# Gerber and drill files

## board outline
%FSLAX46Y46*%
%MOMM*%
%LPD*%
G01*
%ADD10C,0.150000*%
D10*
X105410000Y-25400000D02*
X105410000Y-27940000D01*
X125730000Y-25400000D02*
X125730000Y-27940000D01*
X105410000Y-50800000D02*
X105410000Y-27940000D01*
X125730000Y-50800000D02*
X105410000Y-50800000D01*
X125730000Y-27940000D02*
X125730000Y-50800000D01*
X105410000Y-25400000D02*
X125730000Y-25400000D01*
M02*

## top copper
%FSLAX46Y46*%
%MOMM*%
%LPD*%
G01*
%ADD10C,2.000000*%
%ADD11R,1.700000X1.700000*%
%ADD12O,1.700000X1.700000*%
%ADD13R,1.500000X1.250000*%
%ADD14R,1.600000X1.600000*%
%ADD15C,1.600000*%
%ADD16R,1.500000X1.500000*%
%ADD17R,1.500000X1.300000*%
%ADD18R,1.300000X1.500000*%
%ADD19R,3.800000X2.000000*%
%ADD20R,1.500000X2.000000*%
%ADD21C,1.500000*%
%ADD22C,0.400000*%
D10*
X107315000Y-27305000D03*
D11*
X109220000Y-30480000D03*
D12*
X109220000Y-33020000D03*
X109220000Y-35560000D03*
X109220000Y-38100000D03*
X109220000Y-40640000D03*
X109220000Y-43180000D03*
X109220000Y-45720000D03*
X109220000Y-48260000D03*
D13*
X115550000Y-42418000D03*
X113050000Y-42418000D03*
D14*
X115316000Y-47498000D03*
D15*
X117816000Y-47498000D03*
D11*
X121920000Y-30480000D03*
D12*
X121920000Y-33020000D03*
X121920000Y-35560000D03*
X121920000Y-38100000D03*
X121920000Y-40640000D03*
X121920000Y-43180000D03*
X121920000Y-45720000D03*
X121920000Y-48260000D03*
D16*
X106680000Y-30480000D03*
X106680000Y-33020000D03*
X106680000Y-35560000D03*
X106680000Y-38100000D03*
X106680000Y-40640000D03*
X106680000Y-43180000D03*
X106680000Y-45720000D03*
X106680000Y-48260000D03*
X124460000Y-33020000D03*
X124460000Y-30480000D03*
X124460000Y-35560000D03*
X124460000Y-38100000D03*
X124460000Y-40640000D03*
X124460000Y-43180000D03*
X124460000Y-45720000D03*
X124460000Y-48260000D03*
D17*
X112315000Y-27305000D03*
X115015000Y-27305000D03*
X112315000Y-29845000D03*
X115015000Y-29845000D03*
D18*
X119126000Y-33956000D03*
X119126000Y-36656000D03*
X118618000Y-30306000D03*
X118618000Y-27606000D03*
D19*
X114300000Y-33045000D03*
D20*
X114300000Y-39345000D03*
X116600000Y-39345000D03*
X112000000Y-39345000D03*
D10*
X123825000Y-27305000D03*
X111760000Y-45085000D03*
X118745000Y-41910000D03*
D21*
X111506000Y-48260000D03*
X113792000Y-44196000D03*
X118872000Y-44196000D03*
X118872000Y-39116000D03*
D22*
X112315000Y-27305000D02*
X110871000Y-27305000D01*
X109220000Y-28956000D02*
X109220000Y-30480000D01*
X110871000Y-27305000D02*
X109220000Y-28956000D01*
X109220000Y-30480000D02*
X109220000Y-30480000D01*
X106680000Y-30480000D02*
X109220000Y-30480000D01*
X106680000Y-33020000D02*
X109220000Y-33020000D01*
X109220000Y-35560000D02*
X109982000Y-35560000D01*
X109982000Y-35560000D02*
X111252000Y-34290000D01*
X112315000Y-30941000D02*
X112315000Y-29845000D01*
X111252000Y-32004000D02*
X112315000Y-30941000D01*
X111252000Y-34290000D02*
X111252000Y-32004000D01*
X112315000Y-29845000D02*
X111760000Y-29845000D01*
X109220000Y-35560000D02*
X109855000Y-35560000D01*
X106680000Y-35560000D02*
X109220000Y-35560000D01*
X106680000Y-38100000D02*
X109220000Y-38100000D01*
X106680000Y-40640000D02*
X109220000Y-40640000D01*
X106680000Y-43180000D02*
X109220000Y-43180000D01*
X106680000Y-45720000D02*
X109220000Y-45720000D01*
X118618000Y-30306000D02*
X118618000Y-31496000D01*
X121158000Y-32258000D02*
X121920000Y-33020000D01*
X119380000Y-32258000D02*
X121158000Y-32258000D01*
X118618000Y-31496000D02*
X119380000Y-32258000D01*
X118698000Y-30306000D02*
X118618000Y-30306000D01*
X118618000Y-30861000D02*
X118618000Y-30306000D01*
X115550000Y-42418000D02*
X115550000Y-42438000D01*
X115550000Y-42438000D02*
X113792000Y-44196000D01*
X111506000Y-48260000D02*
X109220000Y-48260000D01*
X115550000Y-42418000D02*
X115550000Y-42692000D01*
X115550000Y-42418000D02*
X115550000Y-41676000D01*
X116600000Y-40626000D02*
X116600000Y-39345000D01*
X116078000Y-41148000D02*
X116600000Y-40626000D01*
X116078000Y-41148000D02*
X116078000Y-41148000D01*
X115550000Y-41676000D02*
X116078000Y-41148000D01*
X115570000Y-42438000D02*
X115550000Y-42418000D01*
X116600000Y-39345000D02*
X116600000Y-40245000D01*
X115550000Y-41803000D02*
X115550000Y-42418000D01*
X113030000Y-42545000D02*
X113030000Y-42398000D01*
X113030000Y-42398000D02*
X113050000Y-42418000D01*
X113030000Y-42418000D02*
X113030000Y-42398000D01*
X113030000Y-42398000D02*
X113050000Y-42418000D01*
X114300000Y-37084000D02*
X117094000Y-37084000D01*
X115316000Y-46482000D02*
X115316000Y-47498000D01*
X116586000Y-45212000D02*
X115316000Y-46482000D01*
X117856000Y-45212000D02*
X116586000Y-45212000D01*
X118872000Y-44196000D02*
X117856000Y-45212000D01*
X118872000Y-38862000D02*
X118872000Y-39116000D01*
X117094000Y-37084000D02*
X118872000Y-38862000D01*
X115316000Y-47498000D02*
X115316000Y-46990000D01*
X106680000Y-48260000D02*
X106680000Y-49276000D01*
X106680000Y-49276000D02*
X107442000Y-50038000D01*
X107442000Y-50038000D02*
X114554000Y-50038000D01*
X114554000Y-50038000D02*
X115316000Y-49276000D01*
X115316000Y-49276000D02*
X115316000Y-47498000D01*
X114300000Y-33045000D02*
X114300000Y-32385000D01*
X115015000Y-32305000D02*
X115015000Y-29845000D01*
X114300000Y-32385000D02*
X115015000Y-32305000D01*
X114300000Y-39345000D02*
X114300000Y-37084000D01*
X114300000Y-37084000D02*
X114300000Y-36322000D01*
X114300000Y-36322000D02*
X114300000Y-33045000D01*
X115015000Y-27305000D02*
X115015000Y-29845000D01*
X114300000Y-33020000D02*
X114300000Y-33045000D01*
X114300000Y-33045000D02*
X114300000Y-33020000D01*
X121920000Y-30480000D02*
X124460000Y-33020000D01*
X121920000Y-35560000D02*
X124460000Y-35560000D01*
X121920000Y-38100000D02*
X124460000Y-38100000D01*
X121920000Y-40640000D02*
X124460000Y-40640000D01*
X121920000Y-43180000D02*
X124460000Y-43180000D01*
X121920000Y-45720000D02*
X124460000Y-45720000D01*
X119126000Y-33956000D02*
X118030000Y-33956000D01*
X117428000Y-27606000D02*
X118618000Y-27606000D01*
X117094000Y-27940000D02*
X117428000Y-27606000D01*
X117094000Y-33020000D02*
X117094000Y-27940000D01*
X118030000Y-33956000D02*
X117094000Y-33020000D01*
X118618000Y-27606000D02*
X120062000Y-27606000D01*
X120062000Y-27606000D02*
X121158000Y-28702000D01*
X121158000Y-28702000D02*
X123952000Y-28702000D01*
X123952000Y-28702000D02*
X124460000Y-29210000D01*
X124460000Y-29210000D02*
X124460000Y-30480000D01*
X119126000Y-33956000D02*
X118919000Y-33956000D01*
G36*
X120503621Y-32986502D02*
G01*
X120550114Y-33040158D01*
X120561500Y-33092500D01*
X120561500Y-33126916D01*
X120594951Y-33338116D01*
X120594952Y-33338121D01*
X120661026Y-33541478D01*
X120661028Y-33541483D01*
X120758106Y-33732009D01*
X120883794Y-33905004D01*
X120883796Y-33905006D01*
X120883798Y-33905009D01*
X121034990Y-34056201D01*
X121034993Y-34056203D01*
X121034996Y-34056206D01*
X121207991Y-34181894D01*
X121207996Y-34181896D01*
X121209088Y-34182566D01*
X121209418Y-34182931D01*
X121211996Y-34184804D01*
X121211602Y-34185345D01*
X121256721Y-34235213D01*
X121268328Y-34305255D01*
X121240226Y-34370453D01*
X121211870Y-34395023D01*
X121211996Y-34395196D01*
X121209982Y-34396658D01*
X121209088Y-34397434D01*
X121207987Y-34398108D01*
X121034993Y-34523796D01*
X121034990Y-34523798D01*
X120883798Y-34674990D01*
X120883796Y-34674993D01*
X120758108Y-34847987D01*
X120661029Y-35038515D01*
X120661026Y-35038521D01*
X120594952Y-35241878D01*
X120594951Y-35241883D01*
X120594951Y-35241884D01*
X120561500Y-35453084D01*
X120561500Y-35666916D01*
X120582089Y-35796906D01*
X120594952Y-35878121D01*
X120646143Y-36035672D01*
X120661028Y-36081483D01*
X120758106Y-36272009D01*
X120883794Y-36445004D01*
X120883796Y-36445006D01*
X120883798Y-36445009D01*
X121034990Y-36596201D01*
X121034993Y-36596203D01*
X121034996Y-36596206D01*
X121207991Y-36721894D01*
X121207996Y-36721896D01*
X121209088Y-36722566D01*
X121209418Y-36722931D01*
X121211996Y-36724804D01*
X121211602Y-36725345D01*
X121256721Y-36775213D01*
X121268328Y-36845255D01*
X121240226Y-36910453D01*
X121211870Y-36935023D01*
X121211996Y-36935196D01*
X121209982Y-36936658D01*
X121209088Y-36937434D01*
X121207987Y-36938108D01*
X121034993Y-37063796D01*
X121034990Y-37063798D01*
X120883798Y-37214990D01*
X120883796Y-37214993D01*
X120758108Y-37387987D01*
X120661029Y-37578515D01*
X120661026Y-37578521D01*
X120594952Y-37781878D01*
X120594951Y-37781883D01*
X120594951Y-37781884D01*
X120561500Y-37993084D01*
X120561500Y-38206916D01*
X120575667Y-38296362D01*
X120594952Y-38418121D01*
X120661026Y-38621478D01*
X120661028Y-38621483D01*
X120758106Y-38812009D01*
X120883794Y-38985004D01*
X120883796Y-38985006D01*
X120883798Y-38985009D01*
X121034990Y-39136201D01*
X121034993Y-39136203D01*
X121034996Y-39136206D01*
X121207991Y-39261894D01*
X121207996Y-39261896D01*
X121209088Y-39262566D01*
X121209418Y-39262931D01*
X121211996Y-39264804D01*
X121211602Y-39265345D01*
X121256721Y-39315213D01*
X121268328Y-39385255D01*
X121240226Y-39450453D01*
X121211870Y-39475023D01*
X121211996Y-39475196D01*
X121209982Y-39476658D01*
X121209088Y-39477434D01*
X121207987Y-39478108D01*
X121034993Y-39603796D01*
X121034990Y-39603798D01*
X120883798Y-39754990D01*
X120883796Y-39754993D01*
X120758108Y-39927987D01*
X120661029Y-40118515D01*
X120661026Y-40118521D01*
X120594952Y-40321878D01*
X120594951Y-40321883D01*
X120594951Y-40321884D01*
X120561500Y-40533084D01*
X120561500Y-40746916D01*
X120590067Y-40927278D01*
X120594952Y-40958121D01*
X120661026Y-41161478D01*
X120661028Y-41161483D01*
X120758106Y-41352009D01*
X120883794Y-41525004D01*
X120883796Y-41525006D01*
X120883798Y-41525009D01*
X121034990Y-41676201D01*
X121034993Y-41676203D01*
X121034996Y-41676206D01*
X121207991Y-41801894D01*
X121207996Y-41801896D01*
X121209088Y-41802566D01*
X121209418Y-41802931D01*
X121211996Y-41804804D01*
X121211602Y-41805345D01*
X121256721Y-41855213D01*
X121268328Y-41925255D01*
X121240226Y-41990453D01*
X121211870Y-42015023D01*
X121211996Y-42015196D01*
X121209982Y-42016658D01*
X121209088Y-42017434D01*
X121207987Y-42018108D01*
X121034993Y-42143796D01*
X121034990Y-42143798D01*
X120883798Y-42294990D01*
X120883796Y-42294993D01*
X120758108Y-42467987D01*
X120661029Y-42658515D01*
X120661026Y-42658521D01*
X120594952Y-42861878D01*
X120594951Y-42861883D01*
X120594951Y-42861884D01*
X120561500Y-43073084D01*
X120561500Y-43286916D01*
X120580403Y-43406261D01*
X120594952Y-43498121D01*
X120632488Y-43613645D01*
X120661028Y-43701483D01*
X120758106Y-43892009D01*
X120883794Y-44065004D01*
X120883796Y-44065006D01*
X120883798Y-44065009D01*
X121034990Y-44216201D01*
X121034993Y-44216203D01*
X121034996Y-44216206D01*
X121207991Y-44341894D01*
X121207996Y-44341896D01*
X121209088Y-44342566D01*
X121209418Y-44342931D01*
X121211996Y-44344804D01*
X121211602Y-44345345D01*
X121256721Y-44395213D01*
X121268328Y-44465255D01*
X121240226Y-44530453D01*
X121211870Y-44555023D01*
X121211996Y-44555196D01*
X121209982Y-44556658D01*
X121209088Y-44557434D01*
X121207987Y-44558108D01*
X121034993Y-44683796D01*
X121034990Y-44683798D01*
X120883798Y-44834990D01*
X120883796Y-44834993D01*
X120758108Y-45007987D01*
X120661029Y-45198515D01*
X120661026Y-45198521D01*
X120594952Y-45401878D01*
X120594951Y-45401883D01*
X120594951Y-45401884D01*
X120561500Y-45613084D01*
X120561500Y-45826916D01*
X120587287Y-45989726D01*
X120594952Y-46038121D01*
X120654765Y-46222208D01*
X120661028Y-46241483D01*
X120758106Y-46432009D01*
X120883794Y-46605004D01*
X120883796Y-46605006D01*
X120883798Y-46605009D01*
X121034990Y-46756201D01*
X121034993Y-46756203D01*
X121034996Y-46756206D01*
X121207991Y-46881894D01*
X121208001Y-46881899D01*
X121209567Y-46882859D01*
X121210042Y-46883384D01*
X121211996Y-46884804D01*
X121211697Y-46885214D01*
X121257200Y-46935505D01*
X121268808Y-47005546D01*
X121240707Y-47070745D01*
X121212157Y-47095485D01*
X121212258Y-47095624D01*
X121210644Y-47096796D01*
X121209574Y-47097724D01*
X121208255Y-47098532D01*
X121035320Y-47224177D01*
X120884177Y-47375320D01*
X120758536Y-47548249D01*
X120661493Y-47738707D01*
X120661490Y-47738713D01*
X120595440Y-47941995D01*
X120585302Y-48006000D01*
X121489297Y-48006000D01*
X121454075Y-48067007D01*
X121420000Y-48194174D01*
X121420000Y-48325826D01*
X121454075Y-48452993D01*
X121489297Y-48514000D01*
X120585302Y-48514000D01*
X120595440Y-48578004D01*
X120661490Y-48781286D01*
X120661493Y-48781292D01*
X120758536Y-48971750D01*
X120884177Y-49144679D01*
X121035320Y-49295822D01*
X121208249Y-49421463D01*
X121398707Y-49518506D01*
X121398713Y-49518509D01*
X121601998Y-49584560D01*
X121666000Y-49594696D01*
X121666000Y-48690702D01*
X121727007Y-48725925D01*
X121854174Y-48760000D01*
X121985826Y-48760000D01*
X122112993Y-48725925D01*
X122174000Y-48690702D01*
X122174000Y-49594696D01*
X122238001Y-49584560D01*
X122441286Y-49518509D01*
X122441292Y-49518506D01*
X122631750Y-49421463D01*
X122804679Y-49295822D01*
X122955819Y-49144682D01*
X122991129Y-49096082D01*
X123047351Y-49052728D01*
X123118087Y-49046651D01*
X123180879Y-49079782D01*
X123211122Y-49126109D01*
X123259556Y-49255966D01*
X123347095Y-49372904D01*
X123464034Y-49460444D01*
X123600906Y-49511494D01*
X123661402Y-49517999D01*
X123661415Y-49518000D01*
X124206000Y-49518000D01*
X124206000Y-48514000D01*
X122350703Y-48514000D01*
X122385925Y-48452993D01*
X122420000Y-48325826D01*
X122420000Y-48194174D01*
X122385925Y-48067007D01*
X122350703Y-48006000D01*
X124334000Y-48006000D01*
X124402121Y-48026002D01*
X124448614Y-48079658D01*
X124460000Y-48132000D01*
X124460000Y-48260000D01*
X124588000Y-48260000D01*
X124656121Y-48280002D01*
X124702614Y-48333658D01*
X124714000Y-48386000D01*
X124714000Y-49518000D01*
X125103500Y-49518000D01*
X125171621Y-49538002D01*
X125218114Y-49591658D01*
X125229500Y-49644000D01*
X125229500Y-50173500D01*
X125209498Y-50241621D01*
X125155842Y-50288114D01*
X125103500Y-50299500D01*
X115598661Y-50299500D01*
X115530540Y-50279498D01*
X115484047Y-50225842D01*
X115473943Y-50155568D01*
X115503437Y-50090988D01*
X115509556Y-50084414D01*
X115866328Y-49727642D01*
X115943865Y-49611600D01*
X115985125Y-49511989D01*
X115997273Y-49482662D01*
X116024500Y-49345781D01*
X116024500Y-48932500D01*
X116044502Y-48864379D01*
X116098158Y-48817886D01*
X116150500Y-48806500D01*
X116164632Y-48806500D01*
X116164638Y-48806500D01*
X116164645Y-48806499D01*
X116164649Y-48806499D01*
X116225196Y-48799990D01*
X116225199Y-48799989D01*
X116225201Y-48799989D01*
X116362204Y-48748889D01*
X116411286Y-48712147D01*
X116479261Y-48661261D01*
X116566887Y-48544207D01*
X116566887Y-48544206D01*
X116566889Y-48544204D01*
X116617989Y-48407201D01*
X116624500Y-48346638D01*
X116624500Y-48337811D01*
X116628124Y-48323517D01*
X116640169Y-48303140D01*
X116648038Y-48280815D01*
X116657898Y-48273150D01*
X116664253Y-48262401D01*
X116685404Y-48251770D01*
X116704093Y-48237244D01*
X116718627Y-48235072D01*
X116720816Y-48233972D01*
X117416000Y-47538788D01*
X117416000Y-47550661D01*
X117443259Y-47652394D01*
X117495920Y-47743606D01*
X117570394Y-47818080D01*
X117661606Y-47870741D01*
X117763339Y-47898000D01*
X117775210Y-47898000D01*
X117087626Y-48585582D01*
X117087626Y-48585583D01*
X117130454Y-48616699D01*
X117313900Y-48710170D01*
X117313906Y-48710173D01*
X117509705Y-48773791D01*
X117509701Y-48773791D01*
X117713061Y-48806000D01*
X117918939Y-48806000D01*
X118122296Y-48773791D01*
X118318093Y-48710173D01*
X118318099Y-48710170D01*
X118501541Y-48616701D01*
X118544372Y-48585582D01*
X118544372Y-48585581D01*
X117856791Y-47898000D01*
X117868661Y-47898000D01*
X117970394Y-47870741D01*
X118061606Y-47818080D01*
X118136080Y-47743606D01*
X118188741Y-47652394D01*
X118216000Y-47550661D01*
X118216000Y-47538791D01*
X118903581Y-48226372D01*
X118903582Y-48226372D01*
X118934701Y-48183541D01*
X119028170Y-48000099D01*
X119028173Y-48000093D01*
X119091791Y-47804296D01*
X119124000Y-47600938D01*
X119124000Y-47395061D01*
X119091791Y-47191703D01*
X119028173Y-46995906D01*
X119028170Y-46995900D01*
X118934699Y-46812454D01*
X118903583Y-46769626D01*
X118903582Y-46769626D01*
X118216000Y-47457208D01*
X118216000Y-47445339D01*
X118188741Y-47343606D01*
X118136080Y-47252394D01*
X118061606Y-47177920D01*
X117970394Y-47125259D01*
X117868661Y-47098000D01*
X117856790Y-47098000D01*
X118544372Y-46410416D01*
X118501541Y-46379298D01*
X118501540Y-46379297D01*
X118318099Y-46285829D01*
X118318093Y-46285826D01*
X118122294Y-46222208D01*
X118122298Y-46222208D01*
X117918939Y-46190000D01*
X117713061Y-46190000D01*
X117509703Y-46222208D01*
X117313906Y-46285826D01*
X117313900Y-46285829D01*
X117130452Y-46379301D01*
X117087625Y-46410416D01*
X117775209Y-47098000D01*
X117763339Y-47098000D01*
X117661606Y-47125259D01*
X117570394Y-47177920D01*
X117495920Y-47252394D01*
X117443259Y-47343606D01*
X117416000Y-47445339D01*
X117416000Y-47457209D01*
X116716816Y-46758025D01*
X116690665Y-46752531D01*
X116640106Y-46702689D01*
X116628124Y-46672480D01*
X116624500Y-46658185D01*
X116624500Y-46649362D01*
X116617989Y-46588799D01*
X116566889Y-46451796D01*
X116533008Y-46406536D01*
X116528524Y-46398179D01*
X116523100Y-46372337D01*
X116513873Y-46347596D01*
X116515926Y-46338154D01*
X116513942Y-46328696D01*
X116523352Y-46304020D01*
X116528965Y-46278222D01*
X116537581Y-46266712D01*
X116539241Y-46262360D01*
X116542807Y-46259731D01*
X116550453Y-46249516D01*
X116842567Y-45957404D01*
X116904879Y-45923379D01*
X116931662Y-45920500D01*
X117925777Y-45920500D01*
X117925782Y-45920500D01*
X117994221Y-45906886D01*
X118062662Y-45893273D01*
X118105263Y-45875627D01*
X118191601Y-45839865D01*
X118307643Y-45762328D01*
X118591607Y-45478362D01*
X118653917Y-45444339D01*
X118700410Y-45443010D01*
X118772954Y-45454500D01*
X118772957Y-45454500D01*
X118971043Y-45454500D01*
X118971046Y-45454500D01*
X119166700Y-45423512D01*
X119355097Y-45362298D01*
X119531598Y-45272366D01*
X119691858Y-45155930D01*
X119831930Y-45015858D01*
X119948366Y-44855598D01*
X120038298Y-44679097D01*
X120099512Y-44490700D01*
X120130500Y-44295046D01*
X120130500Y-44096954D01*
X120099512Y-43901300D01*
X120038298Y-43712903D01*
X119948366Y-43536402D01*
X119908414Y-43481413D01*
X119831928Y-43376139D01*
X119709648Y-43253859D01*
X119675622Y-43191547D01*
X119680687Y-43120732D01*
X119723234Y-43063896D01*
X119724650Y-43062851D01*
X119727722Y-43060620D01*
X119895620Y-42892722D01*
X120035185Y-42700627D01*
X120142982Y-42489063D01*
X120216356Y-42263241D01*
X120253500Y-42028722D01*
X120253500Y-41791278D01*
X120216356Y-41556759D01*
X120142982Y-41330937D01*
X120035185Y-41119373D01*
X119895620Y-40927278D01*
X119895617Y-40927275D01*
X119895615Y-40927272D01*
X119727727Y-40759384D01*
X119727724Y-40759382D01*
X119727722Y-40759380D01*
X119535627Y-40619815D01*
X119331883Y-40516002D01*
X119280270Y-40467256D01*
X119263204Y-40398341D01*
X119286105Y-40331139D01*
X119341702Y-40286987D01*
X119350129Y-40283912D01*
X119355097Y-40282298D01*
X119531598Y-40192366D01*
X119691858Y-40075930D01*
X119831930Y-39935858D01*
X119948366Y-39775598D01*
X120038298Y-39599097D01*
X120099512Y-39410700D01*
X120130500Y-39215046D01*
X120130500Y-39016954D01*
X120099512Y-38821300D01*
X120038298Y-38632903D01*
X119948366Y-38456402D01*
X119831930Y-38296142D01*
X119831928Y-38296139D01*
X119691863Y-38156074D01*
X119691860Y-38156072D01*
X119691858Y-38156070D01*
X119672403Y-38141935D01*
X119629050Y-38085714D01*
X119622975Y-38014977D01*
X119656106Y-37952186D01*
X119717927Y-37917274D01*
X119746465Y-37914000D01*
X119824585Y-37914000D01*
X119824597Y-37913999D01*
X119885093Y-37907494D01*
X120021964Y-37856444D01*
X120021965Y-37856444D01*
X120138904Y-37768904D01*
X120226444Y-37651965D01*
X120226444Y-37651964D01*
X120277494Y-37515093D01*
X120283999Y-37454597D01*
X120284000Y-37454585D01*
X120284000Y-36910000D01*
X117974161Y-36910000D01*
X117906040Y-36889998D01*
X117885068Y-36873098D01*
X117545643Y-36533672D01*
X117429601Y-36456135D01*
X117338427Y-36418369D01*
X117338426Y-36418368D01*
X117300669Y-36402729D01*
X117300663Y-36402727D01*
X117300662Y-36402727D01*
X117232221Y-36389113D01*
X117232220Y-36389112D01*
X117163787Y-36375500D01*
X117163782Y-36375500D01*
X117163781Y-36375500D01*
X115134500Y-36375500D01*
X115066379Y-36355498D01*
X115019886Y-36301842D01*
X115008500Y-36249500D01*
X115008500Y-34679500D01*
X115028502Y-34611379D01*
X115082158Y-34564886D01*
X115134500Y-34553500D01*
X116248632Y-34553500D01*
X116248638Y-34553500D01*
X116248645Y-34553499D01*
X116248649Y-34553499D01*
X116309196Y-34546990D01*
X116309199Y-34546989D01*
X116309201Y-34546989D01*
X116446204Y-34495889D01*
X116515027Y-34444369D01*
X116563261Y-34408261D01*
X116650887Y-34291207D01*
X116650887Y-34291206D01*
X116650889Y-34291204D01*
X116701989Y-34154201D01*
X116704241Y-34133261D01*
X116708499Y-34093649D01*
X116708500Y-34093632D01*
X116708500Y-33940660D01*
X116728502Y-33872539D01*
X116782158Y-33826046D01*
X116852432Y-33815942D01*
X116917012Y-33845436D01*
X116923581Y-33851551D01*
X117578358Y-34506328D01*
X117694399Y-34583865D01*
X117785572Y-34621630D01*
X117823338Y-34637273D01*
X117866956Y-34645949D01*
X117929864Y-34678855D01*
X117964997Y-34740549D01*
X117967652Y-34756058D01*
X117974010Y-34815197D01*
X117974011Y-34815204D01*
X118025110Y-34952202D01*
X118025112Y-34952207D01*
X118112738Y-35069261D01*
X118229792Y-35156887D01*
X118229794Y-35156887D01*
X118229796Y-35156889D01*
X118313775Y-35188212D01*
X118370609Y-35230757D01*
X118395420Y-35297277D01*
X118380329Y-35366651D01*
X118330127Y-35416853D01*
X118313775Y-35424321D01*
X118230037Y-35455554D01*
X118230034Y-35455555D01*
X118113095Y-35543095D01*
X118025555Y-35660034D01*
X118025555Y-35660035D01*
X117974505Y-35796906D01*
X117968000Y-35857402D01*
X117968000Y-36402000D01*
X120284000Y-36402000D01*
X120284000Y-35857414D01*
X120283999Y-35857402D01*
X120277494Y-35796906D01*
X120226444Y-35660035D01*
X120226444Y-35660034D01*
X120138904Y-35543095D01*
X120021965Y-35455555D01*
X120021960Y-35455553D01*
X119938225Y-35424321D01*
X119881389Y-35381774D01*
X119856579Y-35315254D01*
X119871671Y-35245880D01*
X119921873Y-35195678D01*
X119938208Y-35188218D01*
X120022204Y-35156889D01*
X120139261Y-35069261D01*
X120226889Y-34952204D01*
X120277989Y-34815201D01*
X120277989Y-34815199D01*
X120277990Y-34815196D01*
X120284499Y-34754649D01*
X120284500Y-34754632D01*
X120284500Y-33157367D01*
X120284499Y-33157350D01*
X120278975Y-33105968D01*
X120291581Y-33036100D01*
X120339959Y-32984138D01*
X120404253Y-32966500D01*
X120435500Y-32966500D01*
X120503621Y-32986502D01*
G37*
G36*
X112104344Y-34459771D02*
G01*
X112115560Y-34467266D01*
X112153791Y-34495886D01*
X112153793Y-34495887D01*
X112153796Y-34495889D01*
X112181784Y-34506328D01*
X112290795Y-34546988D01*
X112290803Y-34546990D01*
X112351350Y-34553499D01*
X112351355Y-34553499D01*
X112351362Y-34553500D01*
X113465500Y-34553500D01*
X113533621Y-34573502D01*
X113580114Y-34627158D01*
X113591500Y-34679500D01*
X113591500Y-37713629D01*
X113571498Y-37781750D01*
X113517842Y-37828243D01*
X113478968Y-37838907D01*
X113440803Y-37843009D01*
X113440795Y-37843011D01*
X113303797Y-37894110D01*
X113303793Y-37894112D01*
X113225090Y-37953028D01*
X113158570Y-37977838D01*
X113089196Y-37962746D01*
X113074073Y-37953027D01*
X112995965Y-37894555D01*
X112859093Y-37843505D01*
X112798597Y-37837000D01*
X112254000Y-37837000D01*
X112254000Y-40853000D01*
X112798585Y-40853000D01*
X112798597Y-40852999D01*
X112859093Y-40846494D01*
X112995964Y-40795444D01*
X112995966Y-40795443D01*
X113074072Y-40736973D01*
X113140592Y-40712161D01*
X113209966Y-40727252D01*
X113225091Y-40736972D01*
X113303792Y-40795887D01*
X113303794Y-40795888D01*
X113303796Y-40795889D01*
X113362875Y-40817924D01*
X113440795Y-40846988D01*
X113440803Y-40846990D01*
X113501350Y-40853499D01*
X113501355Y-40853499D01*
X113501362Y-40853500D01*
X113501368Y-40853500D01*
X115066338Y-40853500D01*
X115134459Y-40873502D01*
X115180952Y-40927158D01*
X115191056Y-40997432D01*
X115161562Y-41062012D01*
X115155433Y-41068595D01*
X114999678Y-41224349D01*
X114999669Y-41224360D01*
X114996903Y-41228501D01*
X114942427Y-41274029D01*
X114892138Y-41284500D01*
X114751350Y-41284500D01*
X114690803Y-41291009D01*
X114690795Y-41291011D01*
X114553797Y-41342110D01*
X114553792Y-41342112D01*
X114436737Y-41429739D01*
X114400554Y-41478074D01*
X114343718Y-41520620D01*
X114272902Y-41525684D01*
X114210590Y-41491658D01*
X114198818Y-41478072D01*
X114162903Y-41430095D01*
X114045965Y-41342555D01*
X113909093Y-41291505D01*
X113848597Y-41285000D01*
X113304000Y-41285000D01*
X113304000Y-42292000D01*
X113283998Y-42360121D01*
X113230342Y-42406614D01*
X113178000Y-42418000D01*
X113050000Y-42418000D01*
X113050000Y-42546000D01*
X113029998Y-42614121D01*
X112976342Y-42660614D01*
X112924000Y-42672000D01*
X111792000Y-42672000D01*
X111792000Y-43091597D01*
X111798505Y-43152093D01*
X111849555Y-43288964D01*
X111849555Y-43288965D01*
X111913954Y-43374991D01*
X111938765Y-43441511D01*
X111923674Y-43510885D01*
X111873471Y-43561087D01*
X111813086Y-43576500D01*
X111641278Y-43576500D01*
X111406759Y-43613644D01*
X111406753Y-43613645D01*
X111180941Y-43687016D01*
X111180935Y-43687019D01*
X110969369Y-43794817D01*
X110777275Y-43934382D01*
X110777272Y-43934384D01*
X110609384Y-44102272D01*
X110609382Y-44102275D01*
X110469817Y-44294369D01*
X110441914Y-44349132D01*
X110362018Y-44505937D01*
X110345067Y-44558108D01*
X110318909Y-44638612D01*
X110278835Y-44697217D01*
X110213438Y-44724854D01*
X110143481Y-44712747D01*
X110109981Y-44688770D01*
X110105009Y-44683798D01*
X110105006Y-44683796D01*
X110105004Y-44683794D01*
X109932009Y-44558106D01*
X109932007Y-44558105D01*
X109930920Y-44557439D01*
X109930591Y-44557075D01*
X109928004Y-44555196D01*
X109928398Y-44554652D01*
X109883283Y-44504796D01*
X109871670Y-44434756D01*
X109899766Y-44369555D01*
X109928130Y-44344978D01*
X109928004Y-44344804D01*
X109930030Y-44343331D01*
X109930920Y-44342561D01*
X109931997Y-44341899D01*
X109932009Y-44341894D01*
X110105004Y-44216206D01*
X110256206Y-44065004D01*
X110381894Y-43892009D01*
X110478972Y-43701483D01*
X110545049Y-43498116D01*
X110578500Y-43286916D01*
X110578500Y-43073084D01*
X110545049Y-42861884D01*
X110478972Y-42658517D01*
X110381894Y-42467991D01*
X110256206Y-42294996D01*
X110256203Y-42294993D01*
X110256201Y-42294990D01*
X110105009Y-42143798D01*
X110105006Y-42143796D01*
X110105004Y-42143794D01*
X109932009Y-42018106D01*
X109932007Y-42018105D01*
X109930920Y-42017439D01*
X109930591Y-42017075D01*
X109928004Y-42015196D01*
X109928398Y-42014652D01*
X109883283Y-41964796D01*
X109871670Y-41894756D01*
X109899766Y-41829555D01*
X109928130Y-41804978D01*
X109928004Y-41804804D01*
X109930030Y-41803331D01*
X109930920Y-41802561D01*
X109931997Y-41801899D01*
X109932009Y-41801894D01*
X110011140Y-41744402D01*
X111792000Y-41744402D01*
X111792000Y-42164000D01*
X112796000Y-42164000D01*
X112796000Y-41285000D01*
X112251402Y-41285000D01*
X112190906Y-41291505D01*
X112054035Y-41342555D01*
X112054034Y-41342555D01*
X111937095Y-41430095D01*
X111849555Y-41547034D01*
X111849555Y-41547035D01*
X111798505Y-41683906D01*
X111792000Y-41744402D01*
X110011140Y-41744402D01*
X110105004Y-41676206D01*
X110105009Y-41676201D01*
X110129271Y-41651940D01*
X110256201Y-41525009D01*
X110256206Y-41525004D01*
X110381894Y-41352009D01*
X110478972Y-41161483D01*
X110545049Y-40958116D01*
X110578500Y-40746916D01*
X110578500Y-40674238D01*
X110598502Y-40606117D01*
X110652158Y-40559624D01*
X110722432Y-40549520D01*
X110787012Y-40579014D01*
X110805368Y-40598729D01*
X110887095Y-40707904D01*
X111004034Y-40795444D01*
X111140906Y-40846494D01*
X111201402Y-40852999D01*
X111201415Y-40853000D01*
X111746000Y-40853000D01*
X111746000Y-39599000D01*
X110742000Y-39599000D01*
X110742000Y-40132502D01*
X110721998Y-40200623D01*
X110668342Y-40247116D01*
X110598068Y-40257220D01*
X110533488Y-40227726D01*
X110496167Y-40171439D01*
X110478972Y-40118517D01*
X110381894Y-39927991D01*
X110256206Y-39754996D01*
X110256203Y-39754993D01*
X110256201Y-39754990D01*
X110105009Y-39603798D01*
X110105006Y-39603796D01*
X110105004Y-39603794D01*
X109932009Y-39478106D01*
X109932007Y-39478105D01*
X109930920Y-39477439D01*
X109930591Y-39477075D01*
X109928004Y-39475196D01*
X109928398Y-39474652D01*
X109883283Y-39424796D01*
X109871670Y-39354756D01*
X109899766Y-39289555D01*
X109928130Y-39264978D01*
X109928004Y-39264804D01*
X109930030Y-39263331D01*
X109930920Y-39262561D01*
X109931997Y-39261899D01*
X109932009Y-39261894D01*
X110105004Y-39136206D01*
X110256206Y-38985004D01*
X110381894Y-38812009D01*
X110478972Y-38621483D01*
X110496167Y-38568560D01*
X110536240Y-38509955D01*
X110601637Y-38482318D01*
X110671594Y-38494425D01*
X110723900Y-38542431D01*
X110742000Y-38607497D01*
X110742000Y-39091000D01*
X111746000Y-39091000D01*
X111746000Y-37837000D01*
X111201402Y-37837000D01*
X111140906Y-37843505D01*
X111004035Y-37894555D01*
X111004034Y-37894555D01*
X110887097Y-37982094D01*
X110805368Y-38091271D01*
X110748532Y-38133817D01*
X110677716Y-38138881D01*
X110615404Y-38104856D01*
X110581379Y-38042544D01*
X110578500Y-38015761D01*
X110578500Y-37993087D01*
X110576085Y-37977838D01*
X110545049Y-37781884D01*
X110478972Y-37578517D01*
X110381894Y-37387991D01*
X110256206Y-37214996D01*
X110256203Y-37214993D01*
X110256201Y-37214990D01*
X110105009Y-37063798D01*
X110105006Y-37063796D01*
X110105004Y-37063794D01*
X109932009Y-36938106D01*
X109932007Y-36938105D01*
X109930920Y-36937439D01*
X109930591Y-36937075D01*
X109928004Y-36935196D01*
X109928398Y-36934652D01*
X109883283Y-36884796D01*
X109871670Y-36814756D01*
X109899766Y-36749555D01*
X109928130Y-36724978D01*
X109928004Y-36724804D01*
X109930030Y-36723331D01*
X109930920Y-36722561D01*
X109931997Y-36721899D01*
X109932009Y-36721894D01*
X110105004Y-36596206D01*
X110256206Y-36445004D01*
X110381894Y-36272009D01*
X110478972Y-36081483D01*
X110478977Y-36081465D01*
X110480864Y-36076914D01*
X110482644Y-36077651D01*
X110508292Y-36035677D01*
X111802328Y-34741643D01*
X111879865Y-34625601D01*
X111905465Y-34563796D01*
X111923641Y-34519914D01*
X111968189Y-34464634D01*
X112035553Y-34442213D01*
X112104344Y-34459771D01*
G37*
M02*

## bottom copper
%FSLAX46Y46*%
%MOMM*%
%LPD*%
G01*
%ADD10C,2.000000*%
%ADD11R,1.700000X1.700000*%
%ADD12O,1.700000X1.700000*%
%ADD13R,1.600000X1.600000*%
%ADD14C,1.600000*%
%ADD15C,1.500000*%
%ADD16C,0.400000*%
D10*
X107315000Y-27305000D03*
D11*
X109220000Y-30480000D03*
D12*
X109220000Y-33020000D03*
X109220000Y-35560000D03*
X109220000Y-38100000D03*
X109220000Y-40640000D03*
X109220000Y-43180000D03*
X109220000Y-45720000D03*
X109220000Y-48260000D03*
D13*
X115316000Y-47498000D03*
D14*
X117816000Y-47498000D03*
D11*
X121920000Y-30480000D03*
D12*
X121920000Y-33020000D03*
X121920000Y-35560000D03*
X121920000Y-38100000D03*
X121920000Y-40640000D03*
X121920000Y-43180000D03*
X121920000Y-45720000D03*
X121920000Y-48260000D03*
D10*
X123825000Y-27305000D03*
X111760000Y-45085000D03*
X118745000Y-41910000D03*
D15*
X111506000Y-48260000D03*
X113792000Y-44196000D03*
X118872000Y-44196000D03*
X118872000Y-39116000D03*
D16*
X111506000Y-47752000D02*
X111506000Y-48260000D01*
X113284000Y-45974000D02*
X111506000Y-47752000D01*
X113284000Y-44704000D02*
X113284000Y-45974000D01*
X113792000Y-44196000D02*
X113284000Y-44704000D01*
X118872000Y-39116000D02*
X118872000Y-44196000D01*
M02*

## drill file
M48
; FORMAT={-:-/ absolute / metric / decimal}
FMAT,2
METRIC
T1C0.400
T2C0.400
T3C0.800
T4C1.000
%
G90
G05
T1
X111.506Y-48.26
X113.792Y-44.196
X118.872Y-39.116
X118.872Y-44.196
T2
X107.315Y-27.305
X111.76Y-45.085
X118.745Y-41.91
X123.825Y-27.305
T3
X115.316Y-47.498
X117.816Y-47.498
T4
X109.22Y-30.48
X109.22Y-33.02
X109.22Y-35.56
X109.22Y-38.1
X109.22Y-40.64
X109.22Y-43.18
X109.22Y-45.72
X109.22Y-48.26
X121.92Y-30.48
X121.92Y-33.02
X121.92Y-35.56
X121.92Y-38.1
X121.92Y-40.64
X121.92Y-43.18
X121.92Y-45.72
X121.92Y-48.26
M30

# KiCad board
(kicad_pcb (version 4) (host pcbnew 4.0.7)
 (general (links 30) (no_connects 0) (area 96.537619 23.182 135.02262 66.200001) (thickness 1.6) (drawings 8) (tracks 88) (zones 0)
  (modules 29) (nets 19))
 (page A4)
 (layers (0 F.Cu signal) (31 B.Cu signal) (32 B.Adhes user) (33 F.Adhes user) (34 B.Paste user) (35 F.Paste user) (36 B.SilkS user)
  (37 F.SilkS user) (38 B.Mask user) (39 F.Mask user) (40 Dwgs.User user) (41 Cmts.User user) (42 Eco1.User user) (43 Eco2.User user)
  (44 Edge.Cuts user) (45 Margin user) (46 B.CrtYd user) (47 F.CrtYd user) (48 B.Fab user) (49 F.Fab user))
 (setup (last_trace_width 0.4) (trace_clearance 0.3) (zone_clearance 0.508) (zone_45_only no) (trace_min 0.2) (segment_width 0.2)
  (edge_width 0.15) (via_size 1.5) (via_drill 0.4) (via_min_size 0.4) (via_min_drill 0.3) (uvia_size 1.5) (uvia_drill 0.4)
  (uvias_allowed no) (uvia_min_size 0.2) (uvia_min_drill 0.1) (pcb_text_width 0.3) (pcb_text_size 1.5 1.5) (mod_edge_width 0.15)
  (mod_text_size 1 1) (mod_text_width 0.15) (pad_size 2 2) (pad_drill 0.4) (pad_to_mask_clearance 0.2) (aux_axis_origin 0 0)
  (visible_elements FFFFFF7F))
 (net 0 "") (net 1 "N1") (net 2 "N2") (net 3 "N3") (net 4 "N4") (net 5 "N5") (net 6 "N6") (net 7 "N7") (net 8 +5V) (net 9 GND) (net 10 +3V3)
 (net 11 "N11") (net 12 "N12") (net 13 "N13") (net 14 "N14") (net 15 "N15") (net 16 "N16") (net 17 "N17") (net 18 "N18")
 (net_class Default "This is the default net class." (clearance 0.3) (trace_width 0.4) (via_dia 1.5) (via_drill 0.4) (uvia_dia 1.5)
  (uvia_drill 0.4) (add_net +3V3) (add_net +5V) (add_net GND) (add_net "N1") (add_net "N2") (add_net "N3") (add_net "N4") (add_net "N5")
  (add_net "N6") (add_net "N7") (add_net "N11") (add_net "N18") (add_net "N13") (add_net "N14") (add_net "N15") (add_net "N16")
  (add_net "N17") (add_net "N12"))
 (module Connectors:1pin (layer F.Cu) (at 107.315 27.305)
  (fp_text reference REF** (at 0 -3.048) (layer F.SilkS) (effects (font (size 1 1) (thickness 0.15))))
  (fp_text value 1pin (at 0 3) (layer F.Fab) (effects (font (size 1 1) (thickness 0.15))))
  (pad 1 thru_hole circle (at 0 0) (size 2 2) (drill 0.4) (layers *.Cu *.Mask)))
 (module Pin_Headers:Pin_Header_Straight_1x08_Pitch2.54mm (layer F.Cu) (at 109.22 30.48)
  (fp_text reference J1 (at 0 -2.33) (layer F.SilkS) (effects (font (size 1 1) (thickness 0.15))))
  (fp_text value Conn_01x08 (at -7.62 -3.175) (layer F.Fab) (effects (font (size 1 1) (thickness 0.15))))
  (pad 1 thru_hole rect (at 0 0) (size 1.7 1.7) (drill 1) (layers *.Cu *.Mask) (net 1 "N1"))
  (pad 2 thru_hole oval (at 0 2.54) (size 1.7 1.7) (drill 1) (layers *.Cu *.Mask) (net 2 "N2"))
  (pad 3 thru_hole oval (at 0 5.08) (size 1.7 1.7) (drill 1) (layers *.Cu *.Mask) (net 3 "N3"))
  (pad 4 thru_hole oval (at 0 7.62) (size 1.7 1.7) (drill 1) (layers *.Cu *.Mask) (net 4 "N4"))
  (pad 5 thru_hole oval (at 0 10.16) (size 1.7 1.7) (drill 1) (layers *.Cu *.Mask) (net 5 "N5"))
  (pad 6 thru_hole oval (at 0 12.7) (size 1.7 1.7) (drill 1) (layers *.Cu *.Mask) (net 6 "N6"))
  (pad 7 thru_hole oval (at 0 15.24) (size 1.7 1.7) (drill 1) (layers *.Cu *.Mask) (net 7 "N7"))
  (pad 8 thru_hole oval (at 0 17.78) (size 1.7 1.7) (drill 1) (layers *.Cu *.Mask) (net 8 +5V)))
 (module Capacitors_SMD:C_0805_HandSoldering (layer F.Cu) (at 114.3 42.418 180)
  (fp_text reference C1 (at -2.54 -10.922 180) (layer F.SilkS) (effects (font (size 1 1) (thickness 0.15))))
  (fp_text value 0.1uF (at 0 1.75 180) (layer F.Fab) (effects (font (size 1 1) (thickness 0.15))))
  (pad 1 smd rect (at -1.25 0 180) (size 1.5 1.25) (layers F.Cu F.Paste F.Mask) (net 8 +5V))
  (pad 2 smd rect (at 1.25 0 180) (size 1.5 1.25) (layers F.Cu F.Paste F.Mask) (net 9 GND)))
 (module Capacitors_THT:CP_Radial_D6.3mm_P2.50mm (layer F.Cu) (at 115.316 47.498)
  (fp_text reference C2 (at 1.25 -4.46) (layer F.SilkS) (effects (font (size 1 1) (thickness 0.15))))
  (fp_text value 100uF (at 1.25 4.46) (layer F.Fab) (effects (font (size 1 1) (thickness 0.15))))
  (pad 1 thru_hole rect (at 0 0) (size 1.6 1.6) (drill 0.8) (layers *.Cu *.Mask) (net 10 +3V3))
  (pad 2 thru_hole circle (at 2.5 0) (size 1.6 1.6) (drill 0.8) (layers *.Cu *.Mask) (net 9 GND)))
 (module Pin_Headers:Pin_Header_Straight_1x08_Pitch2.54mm (layer F.Cu) (at 121.92 30.48)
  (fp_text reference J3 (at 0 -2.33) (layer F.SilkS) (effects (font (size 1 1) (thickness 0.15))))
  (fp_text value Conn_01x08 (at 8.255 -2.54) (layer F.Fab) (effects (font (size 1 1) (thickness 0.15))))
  (pad 1 thru_hole rect (at 0 0) (size 1.7 1.7) (drill 1) (layers *.Cu *.Mask) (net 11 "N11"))
  (pad 2 thru_hole oval (at 0 2.54) (size 1.7 1.7) (drill 1) (layers *.Cu *.Mask) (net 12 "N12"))
  (pad 3 thru_hole oval (at 0 5.08) (size 1.7 1.7) (drill 1) (layers *.Cu *.Mask) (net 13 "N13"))
  (pad 4 thru_hole oval (at 0 7.62) (size 1.7 1.7) (drill 1) (layers *.Cu *.Mask) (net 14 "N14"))
  (pad 5 thru_hole oval (at 0 10.16) (size 1.7 1.7) (drill 1) (layers *.Cu *.Mask) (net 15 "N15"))
  (pad 6 thru_hole oval (at 0 12.7) (size 1.7 1.7) (drill 1) (layers *.Cu *.Mask) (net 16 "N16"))
  (pad 7 thru_hole oval (at 0 15.24) (size 1.7 1.7) (drill 1) (layers *.Cu *.Mask) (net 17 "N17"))
  (pad 8 thru_hole oval (at 0 17.78) (size 1.7 1.7) (drill 1) (layers *.Cu *.Mask) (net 9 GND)))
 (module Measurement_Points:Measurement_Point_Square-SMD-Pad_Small (layer F.Cu) (at 106.68 30.48)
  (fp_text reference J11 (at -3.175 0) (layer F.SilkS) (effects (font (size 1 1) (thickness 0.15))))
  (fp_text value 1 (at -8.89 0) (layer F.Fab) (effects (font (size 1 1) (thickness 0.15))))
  (pad 1 smd rect (at 0 0) (size 1.5 1.5) (layers F.Cu F.Mask) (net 1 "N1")))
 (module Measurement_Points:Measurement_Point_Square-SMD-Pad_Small (layer F.Cu) (at 106.68 33.02)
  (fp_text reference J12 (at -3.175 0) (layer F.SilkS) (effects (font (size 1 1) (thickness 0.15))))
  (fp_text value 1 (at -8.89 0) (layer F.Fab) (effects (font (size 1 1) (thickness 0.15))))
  (pad 1 smd rect (at 0 0) (size 1.5 1.5) (layers F.Cu F.Mask) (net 2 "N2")))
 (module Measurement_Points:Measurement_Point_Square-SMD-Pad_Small (layer F.Cu) (at 106.68 35.56)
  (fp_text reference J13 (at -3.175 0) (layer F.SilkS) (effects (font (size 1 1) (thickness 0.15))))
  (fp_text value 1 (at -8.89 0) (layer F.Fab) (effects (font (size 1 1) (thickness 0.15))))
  (pad 1 smd rect (at 0 0) (size 1.5 1.5) (layers F.Cu F.Mask) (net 3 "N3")))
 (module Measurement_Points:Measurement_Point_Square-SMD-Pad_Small (layer F.Cu) (at 106.68 38.1)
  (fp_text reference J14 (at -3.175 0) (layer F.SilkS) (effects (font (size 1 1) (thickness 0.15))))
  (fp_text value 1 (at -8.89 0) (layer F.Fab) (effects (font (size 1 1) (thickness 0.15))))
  (pad 1 smd rect (at 0 0) (size 1.5 1.5) (layers F.Cu F.Mask) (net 4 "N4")))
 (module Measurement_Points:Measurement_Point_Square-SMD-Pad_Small (layer F.Cu) (at 106.68 40.64)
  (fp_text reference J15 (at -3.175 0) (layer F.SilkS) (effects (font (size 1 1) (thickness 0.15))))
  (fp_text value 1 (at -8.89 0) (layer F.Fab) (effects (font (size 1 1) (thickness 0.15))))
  (pad 1 smd rect (at 0 0) (size 1.5 1.5) (layers F.Cu F.Mask) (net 5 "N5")))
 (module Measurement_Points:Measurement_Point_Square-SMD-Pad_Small (layer F.Cu) (at 106.68 43.18)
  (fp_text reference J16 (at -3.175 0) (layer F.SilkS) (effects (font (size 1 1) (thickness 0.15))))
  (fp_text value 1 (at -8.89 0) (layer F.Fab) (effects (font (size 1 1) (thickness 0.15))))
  (pad 1 smd rect (at 0 0) (size 1.5 1.5) (layers F.Cu F.Mask) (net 6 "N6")))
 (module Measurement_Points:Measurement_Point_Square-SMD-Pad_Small (layer F.Cu) (at 106.68 45.72)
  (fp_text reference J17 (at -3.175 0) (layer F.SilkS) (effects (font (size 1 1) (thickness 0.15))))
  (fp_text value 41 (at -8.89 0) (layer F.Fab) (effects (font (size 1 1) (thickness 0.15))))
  (pad 1 smd rect (at 0 0) (size 1.5 1.5) (layers F.Cu F.Mask) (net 7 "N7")))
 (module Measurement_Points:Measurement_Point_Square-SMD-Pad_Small (layer F.Cu) (at 106.68 48.26)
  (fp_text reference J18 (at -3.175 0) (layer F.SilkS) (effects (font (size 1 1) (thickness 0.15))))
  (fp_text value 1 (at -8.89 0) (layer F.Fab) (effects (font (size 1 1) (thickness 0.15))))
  (pad 1 smd rect (at 0 0) (size 1.5 1.5) (layers F.Cu F.Mask) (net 10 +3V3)))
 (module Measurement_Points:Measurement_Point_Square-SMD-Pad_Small (layer F.Cu) (at 124.46 33.02)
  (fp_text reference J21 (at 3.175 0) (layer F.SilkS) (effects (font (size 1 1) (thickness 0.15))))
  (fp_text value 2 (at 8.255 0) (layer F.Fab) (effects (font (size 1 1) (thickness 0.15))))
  (pad 1 smd rect (at 0 0) (size 1.5 1.5) (layers F.Cu F.Mask) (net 11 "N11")))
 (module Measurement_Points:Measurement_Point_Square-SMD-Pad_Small (layer F.Cu) (at 124.46 30.48)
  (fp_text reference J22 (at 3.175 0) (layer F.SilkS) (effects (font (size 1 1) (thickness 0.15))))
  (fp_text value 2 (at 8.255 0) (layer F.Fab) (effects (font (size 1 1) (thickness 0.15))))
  (pad 1 smd rect (at 0 0) (size 1.5 1.5) (layers F.Cu F.Mask) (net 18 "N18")))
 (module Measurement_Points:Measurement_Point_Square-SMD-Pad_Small (layer F.Cu) (at 124.46 35.56)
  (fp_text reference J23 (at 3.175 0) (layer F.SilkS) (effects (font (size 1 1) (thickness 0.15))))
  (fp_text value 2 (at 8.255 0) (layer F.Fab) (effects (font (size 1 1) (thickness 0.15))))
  (pad 1 smd rect (at 0 0) (size 1.5 1.5) (layers F.Cu F.Mask) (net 13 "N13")))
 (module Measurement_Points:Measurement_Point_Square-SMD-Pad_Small (layer F.Cu) (at 124.46 38.1)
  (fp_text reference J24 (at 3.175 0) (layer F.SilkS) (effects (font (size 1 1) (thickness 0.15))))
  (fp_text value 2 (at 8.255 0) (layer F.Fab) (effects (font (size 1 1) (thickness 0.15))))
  (pad 1 smd rect (at 0 0) (size 1.5 1.5) (layers F.Cu F.Mask) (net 14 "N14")))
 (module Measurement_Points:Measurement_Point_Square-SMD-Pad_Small (layer F.Cu) (at 124.46 40.64)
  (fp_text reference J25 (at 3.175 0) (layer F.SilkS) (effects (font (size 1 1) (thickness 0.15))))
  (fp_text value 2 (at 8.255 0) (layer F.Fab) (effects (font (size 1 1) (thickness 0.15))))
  (pad 1 smd rect (at 0 0) (size 1.5 1.5) (layers F.Cu F.Mask) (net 15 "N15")))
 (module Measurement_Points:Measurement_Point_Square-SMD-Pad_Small (layer F.Cu) (at 124.46 43.18)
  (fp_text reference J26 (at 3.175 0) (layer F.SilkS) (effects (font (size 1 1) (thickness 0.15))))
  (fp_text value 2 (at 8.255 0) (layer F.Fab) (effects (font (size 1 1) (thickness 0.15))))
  (pad 1 smd rect (at 0 0) (size 1.5 1.5) (layers F.Cu F.Mask) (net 16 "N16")))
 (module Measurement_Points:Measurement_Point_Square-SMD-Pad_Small (layer F.Cu) (at 124.46 45.72)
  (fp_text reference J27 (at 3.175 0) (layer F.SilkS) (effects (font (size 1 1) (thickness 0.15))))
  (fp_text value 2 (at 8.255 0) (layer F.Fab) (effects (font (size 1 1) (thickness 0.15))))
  (pad 1 smd rect (at 0 0) (size 1.5 1.5) (layers F.Cu F.Mask) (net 17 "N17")))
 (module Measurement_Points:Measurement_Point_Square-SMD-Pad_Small (layer F.Cu) (at 124.46 48.26)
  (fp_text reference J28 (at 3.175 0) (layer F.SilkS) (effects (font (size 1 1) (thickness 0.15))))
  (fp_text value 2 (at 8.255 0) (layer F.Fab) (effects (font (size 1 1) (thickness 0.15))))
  (pad 1 smd rect (at 0 0) (size 1.5 1.5) (layers F.Cu F.Mask) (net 9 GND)))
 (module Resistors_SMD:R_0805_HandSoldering (layer F.Cu) (at 113.665 27.305)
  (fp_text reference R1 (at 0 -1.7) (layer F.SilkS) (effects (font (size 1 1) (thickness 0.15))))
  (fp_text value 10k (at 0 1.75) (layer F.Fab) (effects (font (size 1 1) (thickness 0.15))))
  (pad 1 smd rect (at -1.35 0) (size 1.5 1.3) (layers F.Cu F.Paste F.Mask) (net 1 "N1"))
  (pad 2 smd rect (at 1.35 0) (size 1.5 1.3) (layers F.Cu F.Paste F.Mask) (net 10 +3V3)))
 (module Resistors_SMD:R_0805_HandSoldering (layer F.Cu) (at 113.665 29.845)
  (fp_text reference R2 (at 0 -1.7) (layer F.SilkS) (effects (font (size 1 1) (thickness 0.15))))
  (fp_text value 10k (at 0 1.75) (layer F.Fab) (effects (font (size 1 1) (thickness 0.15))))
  (pad 1 smd rect (at -1.35 0) (size 1.5 1.3) (layers F.Cu F.Paste F.Mask) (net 3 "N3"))
  (pad 2 smd rect (at 1.35 0) (size 1.5 1.3) (layers F.Cu F.Paste F.Mask) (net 10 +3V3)))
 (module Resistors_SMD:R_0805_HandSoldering (layer F.Cu) (at 119.126 35.306 270)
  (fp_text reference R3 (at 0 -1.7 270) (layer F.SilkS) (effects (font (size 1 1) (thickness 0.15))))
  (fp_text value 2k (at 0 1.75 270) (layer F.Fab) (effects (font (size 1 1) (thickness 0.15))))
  (pad 1 smd rect (at -1.35 0 270) (size 1.5 1.3) (layers F.Cu F.Paste F.Mask) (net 18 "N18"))
  (pad 2 smd rect (at 1.35 0 270) (size 1.5 1.3) (layers F.Cu F.Paste F.Mask) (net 9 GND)))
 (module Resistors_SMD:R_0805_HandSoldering (layer F.Cu) (at 118.618 28.956 90)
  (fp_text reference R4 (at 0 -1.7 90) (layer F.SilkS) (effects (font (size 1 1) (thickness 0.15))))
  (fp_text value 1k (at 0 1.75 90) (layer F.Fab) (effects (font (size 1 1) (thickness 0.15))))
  (pad 1 smd rect (at -1.35 0 90) (size 1.5 1.3) (layers F.Cu F.Paste F.Mask) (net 12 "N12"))
  (pad 2 smd rect (at 1.35 0 90) (size 1.5 1.3) (layers F.Cu F.Paste F.Mask) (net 18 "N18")))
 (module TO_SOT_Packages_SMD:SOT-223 (layer F.Cu) (at 114.3 36.195 90)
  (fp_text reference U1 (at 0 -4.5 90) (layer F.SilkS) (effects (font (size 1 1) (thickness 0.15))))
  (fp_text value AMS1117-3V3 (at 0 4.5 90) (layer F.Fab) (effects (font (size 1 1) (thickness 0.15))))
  (pad 4 smd rect (at 3.15 0 90) (size 2 3.8) (layers F.Cu F.Paste F.Mask) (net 10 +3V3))
  (pad 2 smd rect (at -3.15 0 90) (size 2 1.5) (layers F.Cu F.Paste F.Mask) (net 10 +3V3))
  (pad 3 smd rect (at -3.15 2.3 90) (size 2 1.5) (layers F.Cu F.Paste F.Mask) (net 8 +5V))
  (pad 1 smd rect (at -3.15 -2.3 90) (size 2 1.5) (layers F.Cu F.Paste F.Mask) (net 9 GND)))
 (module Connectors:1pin (layer F.Cu) (at 123.825 27.305)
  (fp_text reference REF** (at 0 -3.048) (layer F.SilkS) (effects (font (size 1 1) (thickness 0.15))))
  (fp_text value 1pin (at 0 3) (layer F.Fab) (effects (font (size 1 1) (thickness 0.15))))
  (pad 1 thru_hole circle (at 0 0) (size 2 2) (drill 0.4) (layers *.Cu *.Mask)))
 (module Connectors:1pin (layer F.Cu) (at 111.76 45.085)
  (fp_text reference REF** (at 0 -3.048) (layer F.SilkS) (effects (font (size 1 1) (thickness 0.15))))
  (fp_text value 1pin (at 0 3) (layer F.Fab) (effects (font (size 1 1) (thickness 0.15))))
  (pad 1 thru_hole circle (at 0 0) (size 2 2) (drill 0.4) (layers *.Cu *.Mask)))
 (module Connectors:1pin (layer F.Cu) (at 118.745 41.91)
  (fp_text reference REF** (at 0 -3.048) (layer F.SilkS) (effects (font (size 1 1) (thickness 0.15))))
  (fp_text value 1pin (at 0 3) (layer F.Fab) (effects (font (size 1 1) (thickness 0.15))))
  (pad 1 thru_hole circle (at 0 0) (size 2 2) (drill 0.4) (layers *.Cu *.Mask)))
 (gr_line (start 105.41 25.4) (end 105.41 27.94) (angle 90) (layer Edge.Cuts) (width 0.15))
 (gr_line (start 125.73 25.4) (end 125.73 27.94) (angle 90) (layer Edge.Cuts) (width 0.15))
 (gr_line (start 105.41 50.8) (end 105.41 27.94) (angle 90) (layer Edge.Cuts) (width 0.15))
 (gr_line (start 125.73 50.8) (end 105.41 50.8) (angle 90) (layer Edge.Cuts) (width 0.15))
 (gr_line (start 125.73 27.94) (end 125.73 50.8) (angle 90) (layer Edge.Cuts) (width 0.15))
 (gr_line (start 105.41 25.4) (end 125.73 25.4) (angle 90) (layer Edge.Cuts) (width 0.15))
 (segment (start 112.315 27.305) (end 110.871 27.305) (width 0.4) (layer F.Cu) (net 1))
 (segment (start 109.22 28.956) (end 109.22 30.48) (width 0.4) (layer F.Cu) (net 1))
 (segment (start 110.871 27.305) (end 109.22 28.956) (width 0.4) (layer F.Cu) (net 1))
 (segment (start 109.22 30.48) (end 109.22 30.48) (width 0.4) (layer F.Cu) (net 1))
 (segment (start 106.68 30.48) (end 109.22 30.48) (width 0.4) (layer F.Cu) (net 1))
 (segment (start 106.68 33.02) (end 109.22 33.02) (width 0.4) (layer F.Cu) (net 2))
 (segment (start 109.22 35.56) (end 109.982 35.56) (width 0.4) (layer F.Cu) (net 3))
 (segment (start 109.982 35.56) (end 111.252 34.29) (width 0.4) (layer F.Cu) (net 3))
 (segment (start 112.315 30.941) (end 112.315 29.845) (width 0.4) (layer F.Cu) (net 3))
 (segment (start 111.252 32.004) (end 112.315 30.941) (width 0.4) (layer F.Cu) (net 3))
 (segment (start 111.252 34.29) (end 111.252 32.004) (width 0.4) (layer F.Cu) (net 3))
 (segment (start 112.315 29.845) (end 111.76 29.845) (width 0.4) (layer F.Cu) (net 3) (status 30))
 (segment (start 109.22 35.56) (end 109.855 35.56) (width 0.4) (layer F.Cu) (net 3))
 (segment (start 106.68 35.56) (end 109.22 35.56) (width 0.4) (layer F.Cu) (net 3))
 (segment (start 106.68 38.1) (end 109.22 38.1) (width 0.4) (layer F.Cu) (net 4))
 (segment (start 106.68 40.64) (end 109.22 40.64) (width 0.4) (layer F.Cu) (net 5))
 (segment (start 106.68 43.18) (end 109.22 43.18) (width 0.4) (layer F.Cu) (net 6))
 (segment (start 106.68 45.72) (end 109.22 45.72) (width 0.4) (layer F.Cu) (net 7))
 (segment (start 118.618 30.306) (end 118.618 31.496) (width 0.4) (layer F.Cu) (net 12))
 (segment (start 121.158 32.258) (end 121.92 33.02) (width 0.4) (layer F.Cu) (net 12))
 (segment (start 119.38 32.258) (end 121.158 32.258) (width 0.4) (layer F.Cu) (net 12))
 (segment (start 118.618 31.496) (end 119.38 32.258) (width 0.4) (layer F.Cu) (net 12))
 (segment (start 118.698 30.306) (end 118.618 30.306) (width 0.4) (layer F.Cu) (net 12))
 (segment (start 118.618 30.861) (end 118.618 30.306) (width 0.4) (layer F.Cu) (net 12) (status 30))
 (segment (start 115.55 42.418) (end 115.55 42.438) (width 0.4) (layer F.Cu) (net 8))
 (segment (start 115.55 42.438) (end 113.792 44.196) (width 0.4) (layer F.Cu) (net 8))
 (segment (start 111.506 48.26) (end 109.22 48.26) (width 0.4) (layer F.Cu) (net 8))
 (via (at 111.506 48.26) (size 1.5) (drill 0.4) (layers F.Cu B.Cu) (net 8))
 (segment (start 111.506 47.752) (end 111.506 48.26) (width 0.4) (layer B.Cu) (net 8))
 (segment (start 113.284 45.974) (end 111.506 47.752) (width 0.4) (layer B.Cu) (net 8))
 (segment (start 113.284 44.704) (end 113.284 45.974) (width 0.4) (layer B.Cu) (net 8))
 (segment (start 113.792 44.196) (end 113.284 44.704) (width 0.4) (layer B.Cu) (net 8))
 (via (at 113.792 44.196) (size 1.5) (drill 0.4) (layers F.Cu B.Cu) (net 8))
 (segment (start 115.55 42.418) (end 115.55 42.692) (width 0.4) (layer F.Cu) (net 8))
 (segment (start 115.55 42.418) (end 115.55 41.676) (width 0.4) (layer F.Cu) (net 8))
 (segment (start 116.6 40.626) (end 116.6 39.345) (width 0.4) (layer F.Cu) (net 8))
 (segment (start 116.078 41.148) (end 116.6 40.626) (width 0.4) (layer F.Cu) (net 8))
 (segment (start 116.078 41.148) (end 116.078 41.148) (width 0.4) (layer F.Cu) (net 8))
 (segment (start 115.55 41.676) (end 116.078 41.148) (width 0.4) (layer F.Cu) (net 8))
 (segment (start 115.57 42.438) (end 115.55 42.418) (width 0.4) (layer F.Cu) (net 8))
 (segment (start 116.6 39.345) (end 116.6 40.245) (width 0.4) (layer F.Cu) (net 8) (status 30))
 (segment (start 115.55 41.803) (end 115.55 42.418) (width 0.4) (layer F.Cu) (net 8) (status 30))
 (segment (start 113.03 42.545) (end 113.03 42.398) (width 0.4) (layer F.Cu) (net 9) (status 20))
 (segment (start 113.03 42.398) (end 113.05 42.418) (width 0.4) (layer F.Cu) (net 9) (status 30))
 (segment (start 113.03 42.418) (end 113.03 42.398) (width 0.4) (layer F.Cu) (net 9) (status 30))
 (segment (start 113.03 42.398) (end 113.05 42.418) (width 0.4) (layer F.Cu) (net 9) (status 30))
 (segment (start 114.3 37.084) (end 117.094 37.084) (width 0.4) (layer F.Cu) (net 10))
 (segment (start 115.316 46.482) (end 115.316 47.498) (width 0.4) (layer F.Cu) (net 10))
 (segment (start 116.586 45.212) (end 115.316 46.482) (width 0.4) (layer F.Cu) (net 10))
 (segment (start 117.856 45.212) (end 116.586 45.212) (width 0.4) (layer F.Cu) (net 10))
 (segment (start 118.872 44.196) (end 117.856 45.212) (width 0.4) (layer F.Cu) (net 10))
 (via (at 118.872 44.196) (size 1.5) (drill 0.4) (layers F.Cu B.Cu) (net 10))
 (segment (start 118.872 39.116) (end 118.872 44.196) (width 0.4) (layer B.Cu) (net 10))
 (via (at 118.872 39.116) (size 1.5) (drill 0.4) (layers F.Cu B.Cu) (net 10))
 (segment (start 118.872 38.862) (end 118.872 39.116) (width 0.4) (layer F.Cu) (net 10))
 (segment (start 117.094 37.084) (end 118.872 38.862) (width 0.4) (layer F.Cu) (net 10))
 (segment (start 115.316 47.498) (end 115.316 46.99) (width 0.4) (layer F.Cu) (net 10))
 (segment (start 106.68 48.26) (end 106.68 49.276) (width 0.4) (layer F.Cu) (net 10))
 (segment (start 106.68 49.276) (end 107.442 50.038) (width 0.4) (layer F.Cu) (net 10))
 (segment (start 107.442 50.038) (end 114.554 50.038) (width 0.4) (layer F.Cu) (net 10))
 (segment (start 114.554 50.038) (end 115.316 49.276) (width 0.4) (layer F.Cu) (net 10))
 (segment (start 115.316 49.276) (end 115.316 47.498) (width 0.4) (layer F.Cu) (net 10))
 (segment (start 114.3 33.045) (end 114.3 32.385) (width 0.4) (layer F.Cu) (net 10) (status 30))
 (segment (start 115.015 32.305) (end 115.015 29.845) (width 0.4) (layer F.Cu) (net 10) (status 10))
 (segment (start 114.3 32.385) (end 115.015 32.305) (width 0.4) (layer F.Cu) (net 10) (status 30))
 (segment (start 114.3 39.345) (end 114.3 37.084) (width 0.4) (layer F.Cu) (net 10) (status 30))
 (segment (start 114.3 37.084) (end 114.3 36.322) (width 0.4) (layer F.Cu) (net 10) (status 30))
 (segment (start 114.3 36.322) (end 114.3 33.045) (width 0.4) (layer F.Cu) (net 10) (status 30))
 (segment (start 115.015 27.305) (end 115.015 29.845) (width 0.4) (layer F.Cu) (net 10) (status 20))
 (segment (start 114.3 33.02) (end 114.3 33.045) (width 0.4) (layer F.Cu) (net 10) (status 30))
 (segment (start 114.3 33.045) (end 114.3 33.02) (width 0.4) (layer F.Cu) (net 10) (status 30))
 (segment (start 121.92 30.48) (end 124.46 33.02) (width 0.4) (layer F.Cu) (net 11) (status 20))
 (segment (start 121.92 35.56) (end 124.46 35.56) (width 0.4) (layer F.Cu) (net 13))
 (segment (start 121.92 38.1) (end 124.46 38.1) (width 0.4) (layer F.Cu) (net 14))
 (segment (start 121.92 40.64) (end 124.46 40.64) (width 0.4) (layer F.Cu) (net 15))
 (segment (start 121.92 43.18) (end 124.46 43.18) (width 0.4) (layer F.Cu) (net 16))
 (segment (start 121.92 45.72) (end 124.46 45.72) (width 0.4) (layer F.Cu) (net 17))
 (segment (start 119.126 33.956) (end 118.03 33.956) (width 0.4) (layer F.Cu) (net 18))
 (segment (start 117.428 27.606) (end 118.618 27.606) (width 0.4) (layer F.Cu) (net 18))
 (segment (start 117.094 27.94) (end 117.428 27.606) (width 0.4) (layer F.Cu) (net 18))
 (segment (start 117.094 33.02) (end 117.094 27.94) (width 0.4) (layer F.Cu) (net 18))
 (segment (start 118.03 33.956) (end 117.094 33.02) (width 0.4) (layer F.Cu) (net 18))
 (segment (start 118.618 27.606) (end 120.062 27.606) (width 0.4) (layer F.Cu) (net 18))
 (segment (start 120.062 27.606) (end 121.158 28.702) (width 0.4) (layer F.Cu) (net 18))
 (segment (start 121.158 28.702) (end 123.952 28.702) (width 0.4) (layer F.Cu) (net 18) (status 20))
 (segment (start 123.952 28.702) (end 124.46 29.21) (width 0.4) (layer F.Cu) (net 18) (status 10))
 (segment (start 124.46 29.21) (end 124.46 30.48) (width 0.4) (layer F.Cu) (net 18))
 (segment (start 119.126 33.956) (end 118.919 33.956) (width 0.4) (layer F.Cu) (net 18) (status 30))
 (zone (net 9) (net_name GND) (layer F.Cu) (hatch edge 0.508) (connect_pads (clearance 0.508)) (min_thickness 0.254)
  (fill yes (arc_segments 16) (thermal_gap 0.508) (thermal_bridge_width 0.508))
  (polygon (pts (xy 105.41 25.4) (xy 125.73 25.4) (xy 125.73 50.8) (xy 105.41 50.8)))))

